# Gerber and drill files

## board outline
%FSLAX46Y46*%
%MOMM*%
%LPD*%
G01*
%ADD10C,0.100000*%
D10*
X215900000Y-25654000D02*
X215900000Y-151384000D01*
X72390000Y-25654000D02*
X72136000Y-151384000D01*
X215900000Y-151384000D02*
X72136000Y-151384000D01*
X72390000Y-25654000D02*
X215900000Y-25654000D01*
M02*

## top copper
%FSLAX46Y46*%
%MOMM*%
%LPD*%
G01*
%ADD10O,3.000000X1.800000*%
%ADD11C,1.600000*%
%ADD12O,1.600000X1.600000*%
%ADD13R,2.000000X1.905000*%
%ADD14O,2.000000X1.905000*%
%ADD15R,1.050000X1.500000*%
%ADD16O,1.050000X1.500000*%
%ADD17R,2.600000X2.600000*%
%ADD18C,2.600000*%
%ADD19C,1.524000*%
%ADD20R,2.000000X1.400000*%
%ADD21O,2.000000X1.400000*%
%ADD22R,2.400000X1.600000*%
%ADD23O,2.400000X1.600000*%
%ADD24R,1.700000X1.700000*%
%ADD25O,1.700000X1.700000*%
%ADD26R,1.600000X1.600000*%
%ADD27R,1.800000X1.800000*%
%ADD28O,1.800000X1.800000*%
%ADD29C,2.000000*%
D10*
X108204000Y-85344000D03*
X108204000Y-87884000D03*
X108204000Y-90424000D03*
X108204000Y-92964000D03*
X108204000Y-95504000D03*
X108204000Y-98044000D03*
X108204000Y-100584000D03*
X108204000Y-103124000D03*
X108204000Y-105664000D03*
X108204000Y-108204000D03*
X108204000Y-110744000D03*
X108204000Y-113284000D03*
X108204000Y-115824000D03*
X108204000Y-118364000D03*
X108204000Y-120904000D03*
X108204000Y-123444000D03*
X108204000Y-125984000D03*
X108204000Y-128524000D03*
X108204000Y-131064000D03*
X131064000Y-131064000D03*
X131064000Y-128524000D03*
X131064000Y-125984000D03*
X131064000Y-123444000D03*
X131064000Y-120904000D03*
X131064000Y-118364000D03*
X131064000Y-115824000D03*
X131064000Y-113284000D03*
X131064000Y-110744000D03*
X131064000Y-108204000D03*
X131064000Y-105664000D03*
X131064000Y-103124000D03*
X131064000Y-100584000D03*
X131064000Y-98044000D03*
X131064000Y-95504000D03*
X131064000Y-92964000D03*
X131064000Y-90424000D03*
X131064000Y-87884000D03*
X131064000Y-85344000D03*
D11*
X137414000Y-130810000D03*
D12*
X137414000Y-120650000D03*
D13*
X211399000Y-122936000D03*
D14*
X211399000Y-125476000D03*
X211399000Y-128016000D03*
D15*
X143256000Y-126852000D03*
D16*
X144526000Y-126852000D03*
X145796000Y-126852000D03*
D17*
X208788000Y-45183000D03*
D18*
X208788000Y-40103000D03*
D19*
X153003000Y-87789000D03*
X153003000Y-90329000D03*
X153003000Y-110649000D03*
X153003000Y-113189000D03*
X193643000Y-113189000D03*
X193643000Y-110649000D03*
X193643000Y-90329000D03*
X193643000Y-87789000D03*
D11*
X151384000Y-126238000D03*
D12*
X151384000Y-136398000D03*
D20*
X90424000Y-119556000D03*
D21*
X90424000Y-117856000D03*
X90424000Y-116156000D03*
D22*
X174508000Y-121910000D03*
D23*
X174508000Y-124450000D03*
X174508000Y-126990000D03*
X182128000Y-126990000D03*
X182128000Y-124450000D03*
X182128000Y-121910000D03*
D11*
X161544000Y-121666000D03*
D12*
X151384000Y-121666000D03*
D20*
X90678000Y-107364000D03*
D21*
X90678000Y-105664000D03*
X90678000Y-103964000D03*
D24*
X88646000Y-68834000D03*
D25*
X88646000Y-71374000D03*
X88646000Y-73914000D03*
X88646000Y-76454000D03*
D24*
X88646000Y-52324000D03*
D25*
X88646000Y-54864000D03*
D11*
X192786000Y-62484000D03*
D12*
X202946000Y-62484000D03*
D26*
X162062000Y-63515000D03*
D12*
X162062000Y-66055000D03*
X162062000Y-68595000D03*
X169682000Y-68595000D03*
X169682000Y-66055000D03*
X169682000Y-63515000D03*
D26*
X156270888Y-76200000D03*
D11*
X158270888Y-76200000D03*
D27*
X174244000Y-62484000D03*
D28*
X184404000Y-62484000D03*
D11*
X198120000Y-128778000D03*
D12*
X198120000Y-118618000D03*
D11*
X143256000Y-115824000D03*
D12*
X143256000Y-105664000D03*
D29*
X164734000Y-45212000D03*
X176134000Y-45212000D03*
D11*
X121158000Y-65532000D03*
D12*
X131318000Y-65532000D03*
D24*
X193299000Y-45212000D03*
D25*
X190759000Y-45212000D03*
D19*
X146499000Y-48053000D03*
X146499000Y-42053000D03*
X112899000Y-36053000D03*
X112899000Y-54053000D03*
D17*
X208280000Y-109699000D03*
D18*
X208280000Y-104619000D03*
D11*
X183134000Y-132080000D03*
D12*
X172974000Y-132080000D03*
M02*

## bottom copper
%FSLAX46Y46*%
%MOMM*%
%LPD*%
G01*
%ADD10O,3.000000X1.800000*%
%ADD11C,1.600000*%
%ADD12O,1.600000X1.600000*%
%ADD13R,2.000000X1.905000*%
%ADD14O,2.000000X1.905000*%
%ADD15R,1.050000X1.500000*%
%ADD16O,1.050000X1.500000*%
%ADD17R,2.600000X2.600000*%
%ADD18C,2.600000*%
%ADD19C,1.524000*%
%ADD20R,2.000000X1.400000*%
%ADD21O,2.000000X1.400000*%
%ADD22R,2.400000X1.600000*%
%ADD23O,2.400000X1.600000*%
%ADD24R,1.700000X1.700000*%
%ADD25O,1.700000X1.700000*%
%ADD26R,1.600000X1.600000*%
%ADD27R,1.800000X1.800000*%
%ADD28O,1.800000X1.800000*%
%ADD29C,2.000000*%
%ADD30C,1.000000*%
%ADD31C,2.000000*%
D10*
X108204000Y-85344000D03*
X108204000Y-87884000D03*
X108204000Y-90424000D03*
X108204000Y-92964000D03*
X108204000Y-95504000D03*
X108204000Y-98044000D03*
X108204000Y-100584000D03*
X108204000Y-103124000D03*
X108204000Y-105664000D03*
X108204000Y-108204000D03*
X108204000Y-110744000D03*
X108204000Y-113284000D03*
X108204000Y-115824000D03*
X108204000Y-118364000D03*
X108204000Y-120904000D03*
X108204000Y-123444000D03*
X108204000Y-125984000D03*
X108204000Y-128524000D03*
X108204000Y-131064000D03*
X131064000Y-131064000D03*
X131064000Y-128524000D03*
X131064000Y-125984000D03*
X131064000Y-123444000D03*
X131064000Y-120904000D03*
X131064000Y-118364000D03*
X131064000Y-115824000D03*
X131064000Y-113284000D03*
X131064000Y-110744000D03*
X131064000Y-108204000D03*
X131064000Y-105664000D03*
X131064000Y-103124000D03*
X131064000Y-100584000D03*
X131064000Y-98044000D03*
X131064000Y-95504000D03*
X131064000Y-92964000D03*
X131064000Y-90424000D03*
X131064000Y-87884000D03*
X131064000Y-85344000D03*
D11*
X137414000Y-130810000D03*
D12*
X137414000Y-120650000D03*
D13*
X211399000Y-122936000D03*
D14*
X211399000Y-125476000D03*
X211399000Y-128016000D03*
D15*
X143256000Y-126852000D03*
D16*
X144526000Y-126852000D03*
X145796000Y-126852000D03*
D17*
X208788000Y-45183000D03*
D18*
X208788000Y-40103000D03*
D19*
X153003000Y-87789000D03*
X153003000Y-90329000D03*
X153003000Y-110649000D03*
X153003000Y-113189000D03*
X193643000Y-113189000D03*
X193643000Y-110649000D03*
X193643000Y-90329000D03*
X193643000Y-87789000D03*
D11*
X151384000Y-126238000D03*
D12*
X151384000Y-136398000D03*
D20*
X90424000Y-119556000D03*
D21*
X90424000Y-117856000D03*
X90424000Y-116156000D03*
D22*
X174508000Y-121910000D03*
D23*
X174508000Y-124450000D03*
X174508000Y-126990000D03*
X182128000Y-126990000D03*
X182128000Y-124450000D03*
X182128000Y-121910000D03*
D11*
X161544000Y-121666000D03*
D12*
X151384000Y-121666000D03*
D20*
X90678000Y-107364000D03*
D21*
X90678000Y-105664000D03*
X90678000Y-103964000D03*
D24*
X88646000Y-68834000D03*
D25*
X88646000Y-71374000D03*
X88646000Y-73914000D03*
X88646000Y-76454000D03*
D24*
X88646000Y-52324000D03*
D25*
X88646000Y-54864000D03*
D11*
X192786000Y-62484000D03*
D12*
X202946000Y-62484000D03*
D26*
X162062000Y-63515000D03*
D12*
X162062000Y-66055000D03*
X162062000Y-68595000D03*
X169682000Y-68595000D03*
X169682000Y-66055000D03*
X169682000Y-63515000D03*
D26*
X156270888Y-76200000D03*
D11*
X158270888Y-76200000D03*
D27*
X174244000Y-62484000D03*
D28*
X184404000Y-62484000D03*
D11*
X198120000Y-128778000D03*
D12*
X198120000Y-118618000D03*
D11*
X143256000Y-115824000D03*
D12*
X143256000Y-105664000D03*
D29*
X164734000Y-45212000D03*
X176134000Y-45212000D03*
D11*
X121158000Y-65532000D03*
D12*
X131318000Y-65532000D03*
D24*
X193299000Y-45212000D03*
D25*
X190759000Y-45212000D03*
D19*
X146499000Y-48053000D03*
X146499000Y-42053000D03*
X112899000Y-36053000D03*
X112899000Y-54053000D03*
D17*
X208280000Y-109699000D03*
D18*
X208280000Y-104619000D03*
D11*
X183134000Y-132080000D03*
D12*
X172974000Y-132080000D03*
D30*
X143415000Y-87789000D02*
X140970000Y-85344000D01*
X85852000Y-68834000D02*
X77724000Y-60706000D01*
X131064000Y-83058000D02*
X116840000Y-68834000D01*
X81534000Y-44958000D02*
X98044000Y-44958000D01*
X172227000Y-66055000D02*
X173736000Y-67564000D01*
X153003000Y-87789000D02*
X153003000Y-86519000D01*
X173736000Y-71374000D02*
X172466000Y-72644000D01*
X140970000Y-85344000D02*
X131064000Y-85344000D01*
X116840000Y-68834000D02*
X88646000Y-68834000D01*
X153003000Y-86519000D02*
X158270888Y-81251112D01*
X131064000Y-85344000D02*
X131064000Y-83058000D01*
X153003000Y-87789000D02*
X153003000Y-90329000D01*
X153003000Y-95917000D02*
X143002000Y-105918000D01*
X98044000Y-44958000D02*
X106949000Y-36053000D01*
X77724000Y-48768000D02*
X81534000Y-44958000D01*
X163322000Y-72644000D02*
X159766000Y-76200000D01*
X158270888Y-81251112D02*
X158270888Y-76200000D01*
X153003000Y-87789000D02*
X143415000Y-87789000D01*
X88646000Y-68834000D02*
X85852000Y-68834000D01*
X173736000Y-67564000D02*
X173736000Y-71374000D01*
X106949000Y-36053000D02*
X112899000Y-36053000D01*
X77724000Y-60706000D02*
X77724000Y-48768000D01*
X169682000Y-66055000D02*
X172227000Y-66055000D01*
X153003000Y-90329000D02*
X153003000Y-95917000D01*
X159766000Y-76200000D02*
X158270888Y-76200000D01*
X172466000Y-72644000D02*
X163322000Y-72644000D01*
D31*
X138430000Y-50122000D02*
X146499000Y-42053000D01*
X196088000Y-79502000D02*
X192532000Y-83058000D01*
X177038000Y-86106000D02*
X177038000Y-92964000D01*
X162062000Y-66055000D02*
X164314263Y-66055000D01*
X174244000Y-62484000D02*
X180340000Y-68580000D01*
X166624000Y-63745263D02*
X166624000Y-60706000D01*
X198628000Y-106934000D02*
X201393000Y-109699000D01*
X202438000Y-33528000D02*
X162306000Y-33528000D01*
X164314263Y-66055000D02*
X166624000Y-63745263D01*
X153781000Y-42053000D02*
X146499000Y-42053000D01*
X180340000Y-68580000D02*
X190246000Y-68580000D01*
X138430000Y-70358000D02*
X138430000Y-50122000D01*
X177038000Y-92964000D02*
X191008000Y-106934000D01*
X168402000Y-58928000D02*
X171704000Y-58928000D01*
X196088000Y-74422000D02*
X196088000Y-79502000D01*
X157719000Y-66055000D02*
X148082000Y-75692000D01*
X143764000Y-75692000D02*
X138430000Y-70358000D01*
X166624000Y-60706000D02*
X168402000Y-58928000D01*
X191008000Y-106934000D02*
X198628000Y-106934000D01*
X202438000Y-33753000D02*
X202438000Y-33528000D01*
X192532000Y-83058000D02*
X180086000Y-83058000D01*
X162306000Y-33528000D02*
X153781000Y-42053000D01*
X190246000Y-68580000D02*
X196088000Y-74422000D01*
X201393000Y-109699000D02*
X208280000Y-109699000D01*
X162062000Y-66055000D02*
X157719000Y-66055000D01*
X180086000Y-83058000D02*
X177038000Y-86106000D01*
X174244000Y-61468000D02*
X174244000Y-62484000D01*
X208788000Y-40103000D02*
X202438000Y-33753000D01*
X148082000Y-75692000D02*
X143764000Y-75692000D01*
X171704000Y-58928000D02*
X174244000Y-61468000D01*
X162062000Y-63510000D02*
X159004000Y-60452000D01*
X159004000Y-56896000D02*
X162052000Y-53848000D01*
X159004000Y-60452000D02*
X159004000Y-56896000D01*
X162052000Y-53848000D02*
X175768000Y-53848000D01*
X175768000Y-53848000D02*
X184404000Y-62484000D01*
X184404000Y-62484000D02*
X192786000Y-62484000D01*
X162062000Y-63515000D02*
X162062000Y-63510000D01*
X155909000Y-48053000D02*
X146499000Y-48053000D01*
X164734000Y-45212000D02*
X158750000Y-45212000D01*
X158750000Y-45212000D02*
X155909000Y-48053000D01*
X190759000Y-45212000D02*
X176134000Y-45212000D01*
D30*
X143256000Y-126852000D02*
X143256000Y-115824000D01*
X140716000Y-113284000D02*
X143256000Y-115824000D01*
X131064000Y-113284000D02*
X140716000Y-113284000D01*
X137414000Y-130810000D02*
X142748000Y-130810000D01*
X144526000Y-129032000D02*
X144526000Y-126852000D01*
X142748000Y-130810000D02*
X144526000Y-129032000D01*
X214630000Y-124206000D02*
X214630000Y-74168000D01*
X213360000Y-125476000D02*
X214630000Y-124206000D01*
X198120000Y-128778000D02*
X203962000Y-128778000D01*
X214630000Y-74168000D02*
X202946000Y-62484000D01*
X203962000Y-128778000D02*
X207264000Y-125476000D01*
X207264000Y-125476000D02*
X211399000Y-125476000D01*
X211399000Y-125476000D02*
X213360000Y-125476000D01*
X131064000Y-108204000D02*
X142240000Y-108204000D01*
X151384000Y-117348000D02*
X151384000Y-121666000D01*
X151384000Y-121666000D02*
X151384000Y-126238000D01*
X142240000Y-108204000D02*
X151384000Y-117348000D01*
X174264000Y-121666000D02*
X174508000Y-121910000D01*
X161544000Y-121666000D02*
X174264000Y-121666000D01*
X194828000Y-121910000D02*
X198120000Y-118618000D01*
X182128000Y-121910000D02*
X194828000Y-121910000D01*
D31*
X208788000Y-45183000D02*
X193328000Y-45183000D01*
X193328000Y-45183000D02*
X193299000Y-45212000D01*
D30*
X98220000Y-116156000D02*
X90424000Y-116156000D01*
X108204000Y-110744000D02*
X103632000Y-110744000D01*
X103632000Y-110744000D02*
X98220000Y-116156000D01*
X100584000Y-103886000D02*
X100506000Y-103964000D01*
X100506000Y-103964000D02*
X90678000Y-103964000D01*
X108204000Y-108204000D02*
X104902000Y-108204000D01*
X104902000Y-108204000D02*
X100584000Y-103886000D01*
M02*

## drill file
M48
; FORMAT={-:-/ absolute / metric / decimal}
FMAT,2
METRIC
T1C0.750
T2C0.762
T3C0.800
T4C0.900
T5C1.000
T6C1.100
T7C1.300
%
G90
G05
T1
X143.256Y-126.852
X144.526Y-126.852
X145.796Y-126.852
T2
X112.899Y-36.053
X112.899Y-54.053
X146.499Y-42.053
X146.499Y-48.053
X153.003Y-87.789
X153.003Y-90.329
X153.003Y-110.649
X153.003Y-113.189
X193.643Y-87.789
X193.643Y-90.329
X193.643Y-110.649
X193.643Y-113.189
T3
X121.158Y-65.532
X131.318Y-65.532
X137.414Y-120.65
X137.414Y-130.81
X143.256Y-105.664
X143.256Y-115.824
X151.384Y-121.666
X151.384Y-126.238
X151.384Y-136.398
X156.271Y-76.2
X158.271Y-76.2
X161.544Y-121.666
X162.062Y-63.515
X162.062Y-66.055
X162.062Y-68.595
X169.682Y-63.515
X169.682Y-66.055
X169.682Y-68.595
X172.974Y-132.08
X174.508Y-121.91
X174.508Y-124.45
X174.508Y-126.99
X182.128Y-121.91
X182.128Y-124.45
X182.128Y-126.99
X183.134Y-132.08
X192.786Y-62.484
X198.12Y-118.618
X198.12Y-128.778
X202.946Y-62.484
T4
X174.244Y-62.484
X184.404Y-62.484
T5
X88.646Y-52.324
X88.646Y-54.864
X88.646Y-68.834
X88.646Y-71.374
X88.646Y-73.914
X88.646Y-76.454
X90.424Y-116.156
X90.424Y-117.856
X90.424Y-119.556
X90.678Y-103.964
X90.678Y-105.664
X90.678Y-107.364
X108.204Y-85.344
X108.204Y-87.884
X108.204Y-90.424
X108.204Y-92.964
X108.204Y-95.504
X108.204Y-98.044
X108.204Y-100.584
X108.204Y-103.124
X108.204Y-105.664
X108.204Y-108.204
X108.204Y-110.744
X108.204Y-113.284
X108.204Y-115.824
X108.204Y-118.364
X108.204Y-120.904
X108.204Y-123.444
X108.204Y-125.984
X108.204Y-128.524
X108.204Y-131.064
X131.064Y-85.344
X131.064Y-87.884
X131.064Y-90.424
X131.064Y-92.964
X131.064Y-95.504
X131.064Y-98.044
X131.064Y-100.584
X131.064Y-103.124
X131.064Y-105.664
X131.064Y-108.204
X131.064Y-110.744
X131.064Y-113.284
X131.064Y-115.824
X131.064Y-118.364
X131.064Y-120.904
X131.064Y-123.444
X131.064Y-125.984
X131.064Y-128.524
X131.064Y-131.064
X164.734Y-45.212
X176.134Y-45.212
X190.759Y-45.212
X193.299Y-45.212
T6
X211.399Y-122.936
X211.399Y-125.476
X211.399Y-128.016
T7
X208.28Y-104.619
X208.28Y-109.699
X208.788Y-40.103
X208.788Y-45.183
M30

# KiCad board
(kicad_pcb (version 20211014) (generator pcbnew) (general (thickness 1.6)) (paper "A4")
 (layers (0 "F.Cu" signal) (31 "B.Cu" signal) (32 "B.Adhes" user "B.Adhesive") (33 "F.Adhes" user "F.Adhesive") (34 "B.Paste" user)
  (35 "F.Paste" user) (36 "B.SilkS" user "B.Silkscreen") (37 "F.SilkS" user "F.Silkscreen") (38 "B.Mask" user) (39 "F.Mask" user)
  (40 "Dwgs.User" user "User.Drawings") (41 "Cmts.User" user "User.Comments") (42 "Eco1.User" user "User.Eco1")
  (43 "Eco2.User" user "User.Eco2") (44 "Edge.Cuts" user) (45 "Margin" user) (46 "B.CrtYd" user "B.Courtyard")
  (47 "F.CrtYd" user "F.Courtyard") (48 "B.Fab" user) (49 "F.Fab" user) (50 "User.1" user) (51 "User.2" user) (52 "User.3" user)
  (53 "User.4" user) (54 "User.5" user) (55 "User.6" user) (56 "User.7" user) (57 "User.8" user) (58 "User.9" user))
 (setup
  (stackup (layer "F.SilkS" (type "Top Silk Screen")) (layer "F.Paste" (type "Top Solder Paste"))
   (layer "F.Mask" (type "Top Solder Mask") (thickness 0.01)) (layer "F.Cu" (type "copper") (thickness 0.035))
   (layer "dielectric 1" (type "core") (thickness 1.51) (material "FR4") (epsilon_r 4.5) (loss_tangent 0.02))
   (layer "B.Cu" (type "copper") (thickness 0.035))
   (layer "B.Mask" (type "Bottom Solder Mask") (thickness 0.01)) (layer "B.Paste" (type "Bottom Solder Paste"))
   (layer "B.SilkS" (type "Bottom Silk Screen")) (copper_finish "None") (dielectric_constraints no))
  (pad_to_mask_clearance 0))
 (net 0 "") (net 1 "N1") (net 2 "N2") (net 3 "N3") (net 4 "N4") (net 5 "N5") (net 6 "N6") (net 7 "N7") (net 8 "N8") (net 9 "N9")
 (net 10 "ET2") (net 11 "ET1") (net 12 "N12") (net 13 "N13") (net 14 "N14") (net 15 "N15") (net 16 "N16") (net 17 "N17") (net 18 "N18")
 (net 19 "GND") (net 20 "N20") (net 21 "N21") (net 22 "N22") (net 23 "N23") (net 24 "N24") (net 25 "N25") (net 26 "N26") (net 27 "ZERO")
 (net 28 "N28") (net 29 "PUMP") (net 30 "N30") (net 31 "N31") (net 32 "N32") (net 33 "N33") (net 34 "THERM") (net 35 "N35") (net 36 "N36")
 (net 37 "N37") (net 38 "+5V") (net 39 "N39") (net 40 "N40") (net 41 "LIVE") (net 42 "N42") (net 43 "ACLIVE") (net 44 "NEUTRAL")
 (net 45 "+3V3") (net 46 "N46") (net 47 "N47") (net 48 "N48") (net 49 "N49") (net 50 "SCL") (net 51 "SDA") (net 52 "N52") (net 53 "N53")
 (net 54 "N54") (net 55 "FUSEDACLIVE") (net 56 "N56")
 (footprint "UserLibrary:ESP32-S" (layer "F.Cu") (at 119.634 108.204)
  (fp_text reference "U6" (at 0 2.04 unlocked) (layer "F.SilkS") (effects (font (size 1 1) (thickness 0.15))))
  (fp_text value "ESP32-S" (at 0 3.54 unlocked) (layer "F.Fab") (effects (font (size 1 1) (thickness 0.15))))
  (pad "1" thru_hole oval (at -11.43 -22.86) (size 3 1.8) (drill 1) (layers *.Cu *.Mask) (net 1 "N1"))
  (pad "2" thru_hole oval (at -11.43 -20.32) (size 3 1.8) (drill 1) (layers *.Cu *.Mask) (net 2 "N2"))
  (pad "3" thru_hole oval (at -11.43 -17.78) (size 3 1.8) (drill 1) (layers *.Cu *.Mask) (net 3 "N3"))
  (pad "4" thru_hole oval (at -11.43 -15.24) (size 3 1.8) (drill 1) (layers *.Cu *.Mask) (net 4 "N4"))
  (pad "5" thru_hole oval (at -11.43 -12.7) (size 3 1.8) (drill 1) (layers *.Cu *.Mask) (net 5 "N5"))
  (pad "6" thru_hole oval (at -11.43 -10.16) (size 3 1.8) (drill 1) (layers *.Cu *.Mask) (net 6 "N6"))
  (pad "7" thru_hole oval (at -11.43 -7.62) (size 3 1.8) (drill 1) (layers *.Cu *.Mask) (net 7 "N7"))
  (pad "8" thru_hole oval (at -11.43 -5.08) (size 3 1.8) (drill 1) (layers *.Cu *.Mask) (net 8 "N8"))
  (pad "9" thru_hole oval (at -11.43 -2.54) (size 3 1.8) (drill 1) (layers *.Cu *.Mask) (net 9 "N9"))
  (pad "10" thru_hole oval (at -11.43 0) (size 3 1.8) (drill 1) (layers *.Cu *.Mask) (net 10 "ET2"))
  (pad "11" thru_hole oval (at -11.43 2.54) (size 3 1.8) (drill 1) (layers *.Cu *.Mask) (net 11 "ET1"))
  (pad "12" thru_hole oval (at -11.43 5.08) (size 3 1.8) (drill 1) (layers *.Cu *.Mask) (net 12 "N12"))
  (pad "13" thru_hole oval (at -11.43 7.62) (size 3 1.8) (drill 1) (layers *.Cu *.Mask) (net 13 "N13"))
  (pad "14" thru_hole oval (at -11.43 10.16) (size 3 1.8) (drill 1) (layers *.Cu *.Mask) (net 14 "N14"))
  (pad "15" thru_hole oval (at -11.43 12.7) (size 3 1.8) (drill 1) (layers *.Cu *.Mask) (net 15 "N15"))
  (pad "16" thru_hole oval (at -11.43 15.24) (size 3 1.8) (drill 1) (layers *.Cu *.Mask) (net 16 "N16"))
  (pad "17" thru_hole oval (at -11.43 17.78) (size 3 1.8) (drill 1) (layers *.Cu *.Mask) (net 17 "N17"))
  (pad "18" thru_hole oval (at -11.43 20.32) (size 3 1.8) (drill 1) (layers *.Cu *.Mask) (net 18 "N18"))
  (pad "19" thru_hole oval (at -11.43 22.86) (size 3 1.8) (drill 1) (layers *.Cu *.Mask) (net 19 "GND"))
  (pad "20" thru_hole oval (at 11.43 22.86) (size 3 1.8) (drill 1) (layers *.Cu *.Mask) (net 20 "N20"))
  (pad "21" thru_hole oval (at 11.43 20.32) (size 3 1.8) (drill 1) (layers *.Cu *.Mask) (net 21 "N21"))
  (pad "22" thru_hole oval (at 11.43 17.78) (size 3 1.8) (drill 1) (layers *.Cu *.Mask) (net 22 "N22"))
  (pad "23" thru_hole oval (at 11.43 15.24) (size 3 1.8) (drill 1) (layers *.Cu *.Mask) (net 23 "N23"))
  (pad "24" thru_hole oval (at 11.43 12.7) (size 3 1.8) (drill 1) (layers *.Cu *.Mask) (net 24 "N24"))
  (pad "25" thru_hole oval (at 11.43 10.16) (size 3 1.8) (drill 1) (layers *.Cu *.Mask) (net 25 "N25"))
  (pad "26" thru_hole oval (at 11.43 7.62) (size 3 1.8) (drill 1) (layers *.Cu *.Mask) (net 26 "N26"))
  (pad "27" thru_hole oval (at 11.43 5.08) (size 3 1.8) (drill 1) (layers *.Cu *.Mask) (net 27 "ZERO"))
  (pad "28" thru_hole oval (at 11.43 2.54) (size 3 1.8) (drill 1) (layers *.Cu *.Mask) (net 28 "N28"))
  (pad "29" thru_hole oval (at 11.43 0) (size 3 1.8) (drill 1) (layers *.Cu *.Mask) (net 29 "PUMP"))
  (pad "30" thru_hole oval (at 11.43 -2.54) (size 3 1.8) (drill 1) (layers *.Cu *.Mask) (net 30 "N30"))
  (pad "31" thru_hole oval (at 11.43 -5.08) (size 3 1.8) (drill 1) (layers *.Cu *.Mask) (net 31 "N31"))
  (pad "32" thru_hole oval (at 11.43 -7.62) (size 3 1.8) (drill 1) (layers *.Cu *.Mask) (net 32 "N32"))
  (pad "33" thru_hole oval (at 11.43 -10.16) (size 3 1.8) (drill 1) (layers *.Cu *.Mask) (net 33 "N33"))
  (pad "34" thru_hole oval (at 11.43 -12.7) (size 3 1.8) (drill 1) (layers *.Cu *.Mask) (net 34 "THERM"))
  (pad "35" thru_hole oval (at 11.43 -15.24) (size 3 1.8) (drill 1) (layers *.Cu *.Mask) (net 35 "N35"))
  (pad "36" thru_hole oval (at 11.43 -17.78) (size 3 1.8) (drill 1) (layers *.Cu *.Mask) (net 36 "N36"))
  (pad "37" thru_hole oval (at 11.43 -20.32) (size 3 1.8) (drill 1) (layers *.Cu *.Mask) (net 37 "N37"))
  (pad "38" thru_hole oval (at 11.43 -22.86) (size 3 1.8) (drill 1) (layers *.Cu *.Mask) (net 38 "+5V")))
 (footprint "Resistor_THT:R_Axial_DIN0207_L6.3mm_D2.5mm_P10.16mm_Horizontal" (layer "F.Cu") (at 137.414 130.81 90)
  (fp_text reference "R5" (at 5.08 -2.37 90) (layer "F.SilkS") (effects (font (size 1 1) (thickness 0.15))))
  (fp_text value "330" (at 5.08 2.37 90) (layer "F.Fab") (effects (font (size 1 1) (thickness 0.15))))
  (pad "1" thru_hole circle (at 0 0 90) (size 1.6 1.6) (drill 0.8) (layers *.Cu *.Mask) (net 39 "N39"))
  (pad "2" thru_hole oval (at 10.16 0 90) (size 1.6 1.6) (drill 0.8) (layers *.Cu *.Mask) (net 19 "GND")))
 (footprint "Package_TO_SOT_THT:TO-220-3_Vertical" (layer "F.Cu") (at 211.399 122.936 -90)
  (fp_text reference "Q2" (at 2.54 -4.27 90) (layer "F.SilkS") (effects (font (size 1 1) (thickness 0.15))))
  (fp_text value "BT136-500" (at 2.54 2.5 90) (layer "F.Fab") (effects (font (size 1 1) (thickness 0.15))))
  (pad "1" thru_hole rect (at 0 0 270) (size 1.905 2) (drill 1.1) (layers *.Cu *.Mask) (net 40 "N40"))
  (pad "2" thru_hole oval (at 2.54 0 270) (size 1.905 2) (drill 1.1) (layers *.Cu *.Mask) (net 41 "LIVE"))
  (pad "3" thru_hole oval (at 5.08 0 270) (size 1.905 2) (drill 1.1) (layers *.Cu *.Mask) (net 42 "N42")))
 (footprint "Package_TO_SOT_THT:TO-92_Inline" (layer "F.Cu") (at 143.256 126.852)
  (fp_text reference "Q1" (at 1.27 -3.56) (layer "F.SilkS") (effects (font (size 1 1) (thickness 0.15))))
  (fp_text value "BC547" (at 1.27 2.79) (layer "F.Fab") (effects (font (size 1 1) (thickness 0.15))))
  (pad "1" thru_hole rect (at 0 0) (size 1.05 1.5) (drill 0.75) (layers *.Cu *.Mask) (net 27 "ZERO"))
  (pad "2" thru_hole oval (at 1.27 0) (size 1.05 1.5) (drill 0.75) (layers *.Cu *.Mask) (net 39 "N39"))
  (pad "3" thru_hole oval (at 2.54 0) (size 1.05 1.5) (drill 0.75) (layers *.Cu *.Mask) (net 19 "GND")))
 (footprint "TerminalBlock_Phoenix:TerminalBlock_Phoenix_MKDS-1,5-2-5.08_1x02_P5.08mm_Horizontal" (layer "F.Cu") (at 208.788 45.183 90)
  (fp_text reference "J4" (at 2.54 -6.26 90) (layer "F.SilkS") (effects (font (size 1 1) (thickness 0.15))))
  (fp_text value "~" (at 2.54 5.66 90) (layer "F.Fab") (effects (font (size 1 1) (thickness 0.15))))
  (pad "1" thru_hole rect (at 0 0 90) (size 2.6 2.6) (drill 1.3) (layers *.Cu *.Mask) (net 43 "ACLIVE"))
  (pad "2" thru_hole circle (at 5.08 0 90) (size 2.6 2.6) (drill 1.3) (layers *.Cu *.Mask) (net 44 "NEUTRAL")))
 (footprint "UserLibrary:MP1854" (layer "F.Cu") (at 150.463 115.729)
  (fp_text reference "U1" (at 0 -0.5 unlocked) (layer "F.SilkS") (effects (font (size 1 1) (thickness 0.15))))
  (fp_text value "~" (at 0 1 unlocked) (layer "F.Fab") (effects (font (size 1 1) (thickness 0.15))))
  (pad "1" thru_hole circle (at 2.54 -27.94) (size 1.524 1.524) (drill 0.762) (layers *.Cu *.Mask) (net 38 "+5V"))
  (pad "2" thru_hole circle (at 2.54 -25.4) (size 1.524 1.524) (drill 0.762) (layers *.Cu *.Mask) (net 38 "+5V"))
  (pad "3" thru_hole circle (at 2.54 -5.08) (size 1.524 1.524) (drill 0.762) (layers *.Cu *.Mask) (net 19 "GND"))
  (pad "4" thru_hole circle (at 2.54 -2.54) (size 1.524 1.524) (drill 0.762) (layers *.Cu *.Mask) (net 19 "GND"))
  (pad "5" thru_hole circle (at 43.18 -2.54) (size 1.524 1.524) (drill 0.762) (layers *.Cu *.Mask) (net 19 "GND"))
  (pad "6" thru_hole circle (at 43.18 -5.08) (size 1.524 1.524) (drill 0.762) (layers *.Cu *.Mask) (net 19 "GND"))
  (pad "7" thru_hole circle (at 43.18 -25.4) (size 1.524 1.524) (drill 0.762) (layers *.Cu *.Mask) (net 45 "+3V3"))
  (pad "8" thru_hole circle (at 43.18 -27.94) (size 1.524 1.524) (drill 0.762) (layers *.Cu *.Mask) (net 45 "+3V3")))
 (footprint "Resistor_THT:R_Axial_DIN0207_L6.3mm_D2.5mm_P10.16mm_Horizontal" (layer "F.Cu") (at 151.384 126.238 -90)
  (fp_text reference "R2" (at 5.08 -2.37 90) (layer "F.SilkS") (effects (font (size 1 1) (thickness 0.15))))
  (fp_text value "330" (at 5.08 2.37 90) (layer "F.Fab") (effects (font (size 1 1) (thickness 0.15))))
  (pad "1" thru_hole circle (at 0 0 270) (size 1.6 1.6) (drill 0.8) (layers *.Cu *.Mask) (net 29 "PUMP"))
  (pad "2" thru_hole oval (at 10.16 0 270) (size 1.6 1.6) (drill 0.8) (layers *.Cu *.Mask) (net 19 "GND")))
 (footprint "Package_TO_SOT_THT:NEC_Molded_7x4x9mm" (layer "F.Cu") (at 90.424 119.556 90)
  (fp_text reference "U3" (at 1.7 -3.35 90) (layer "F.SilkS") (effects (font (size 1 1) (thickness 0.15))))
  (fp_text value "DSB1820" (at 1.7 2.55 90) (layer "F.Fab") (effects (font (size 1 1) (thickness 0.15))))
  (pad "1" thru_hole rect (at 0 0 270) (size 1.4 2) (drill 1) (layers *.Cu *.Mask) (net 45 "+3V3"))
  (pad "2" thru_hole oval (at 1.7 0 270) (size 1.4 2) (drill 1) (layers *.Cu *.Mask) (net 19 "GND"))
  (pad "3" thru_hole oval (at 3.4 0 270) (size 1.4 2) (drill 1) (layers *.Cu *.Mask) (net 11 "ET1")))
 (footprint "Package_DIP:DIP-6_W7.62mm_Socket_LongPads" (layer "F.Cu") (at 174.508 121.91)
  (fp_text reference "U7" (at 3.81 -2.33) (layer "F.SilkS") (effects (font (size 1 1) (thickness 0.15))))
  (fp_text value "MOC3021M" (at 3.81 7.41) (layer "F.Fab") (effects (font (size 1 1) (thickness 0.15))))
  (pad "1" thru_hole rect (at 0 0) (size 2.4 1.6) (drill 0.8) (layers *.Cu *.Mask) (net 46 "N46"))
  (pad "2" thru_hole oval (at 0 2.54) (size 2.4 1.6) (drill 0.8) (layers *.Cu *.Mask) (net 19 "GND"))
  (pad "3" thru_hole oval (at 0 5.08) (size 2.4 1.6) (drill 0.8) (layers *.Cu *.Mask) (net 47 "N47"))
  (pad "4" thru_hole oval (at 7.62 5.08) (size 2.4 1.6) (drill 0.8) (layers *.Cu *.Mask) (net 42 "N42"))
  (pad "5" thru_hole oval (at 7.62 2.54) (size 2.4 1.6) (drill 0.8) (layers *.Cu *.Mask) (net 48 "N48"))
  (pad "6" thru_hole oval (at 7.62 0) (size 2.4 1.6) (drill 0.8) (layers *.Cu *.Mask) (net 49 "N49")))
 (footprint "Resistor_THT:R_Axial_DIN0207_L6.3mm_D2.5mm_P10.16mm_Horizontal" (layer "F.Cu") (at 161.544 121.666 180)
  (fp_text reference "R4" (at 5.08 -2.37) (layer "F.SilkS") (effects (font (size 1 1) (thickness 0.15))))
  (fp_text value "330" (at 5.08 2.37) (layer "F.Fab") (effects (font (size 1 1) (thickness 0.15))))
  (pad "1" thru_hole circle (at 0 0 180) (size 1.6 1.6) (drill 0.8) (layers *.Cu *.Mask) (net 46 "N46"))
  (pad "2" thru_hole oval (at 10.16 0 180) (size 1.6 1.6) (drill 0.8) (layers *.Cu *.Mask) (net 29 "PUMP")))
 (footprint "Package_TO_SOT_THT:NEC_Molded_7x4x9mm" (layer "F.Cu") (at 90.678 107.364 90)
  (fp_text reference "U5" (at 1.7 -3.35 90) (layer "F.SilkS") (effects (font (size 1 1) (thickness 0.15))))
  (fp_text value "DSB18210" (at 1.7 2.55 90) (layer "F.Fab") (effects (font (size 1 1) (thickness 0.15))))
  (pad "1" thru_hole rect (at 0 0 270) (size 1.4 2) (drill 1) (layers *.Cu *.Mask) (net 45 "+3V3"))
  (pad "2" thru_hole oval (at 1.7 0 270) (size 1.4 2) (drill 1) (layers *.Cu *.Mask) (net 19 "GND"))
  (pad "3" thru_hole oval (at 3.4 0 270) (size 1.4 2) (drill 1) (layers *.Cu *.Mask) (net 10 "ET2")))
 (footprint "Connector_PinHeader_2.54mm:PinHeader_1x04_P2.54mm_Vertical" (layer "F.Cu") (at 88.646 68.834)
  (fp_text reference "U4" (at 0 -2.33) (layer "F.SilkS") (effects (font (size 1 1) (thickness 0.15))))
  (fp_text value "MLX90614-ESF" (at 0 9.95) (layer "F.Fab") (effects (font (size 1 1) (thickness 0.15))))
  (pad "1" thru_hole rect (at 0 0) (size 1.7 1.7) (drill 1) (layers *.Cu *.Mask) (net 38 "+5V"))
  (pad "2" thru_hole oval (at 0 2.54) (size 1.7 1.7) (drill 1) (layers *.Cu *.Mask) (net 19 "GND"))
  (pad "3" thru_hole oval (at 0 5.08) (size 1.7 1.7) (drill 1) (layers *.Cu *.Mask) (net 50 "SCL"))
  (pad "4" thru_hole oval (at 0 7.62) (size 1.7 1.7) (drill 1) (layers *.Cu *.Mask) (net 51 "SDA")))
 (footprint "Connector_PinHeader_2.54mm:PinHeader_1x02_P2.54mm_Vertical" (layer "F.Cu") (at 88.646 52.324)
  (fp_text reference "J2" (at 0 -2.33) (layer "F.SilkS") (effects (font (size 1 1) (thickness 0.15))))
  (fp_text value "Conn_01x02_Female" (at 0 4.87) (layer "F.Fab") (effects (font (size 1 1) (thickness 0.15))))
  (pad "1" thru_hole rect (at 0 0) (size 1.7 1.7) (drill 1) (layers *.Cu *.Mask) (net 34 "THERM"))
  (pad "2" thru_hole oval (at 0 2.54) (size 1.7 1.7) (drill 1) (layers *.Cu *.Mask) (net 19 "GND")))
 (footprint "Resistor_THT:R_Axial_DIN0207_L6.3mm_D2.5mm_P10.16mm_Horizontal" (layer "F.Cu") (at 192.786 62.484)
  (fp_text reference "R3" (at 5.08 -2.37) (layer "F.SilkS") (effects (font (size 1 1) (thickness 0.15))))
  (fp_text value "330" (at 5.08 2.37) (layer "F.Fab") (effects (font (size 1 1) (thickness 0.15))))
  (pad "1" thru_hole circle (at 0 0) (size 1.6 1.6) (drill 0.8) (layers *.Cu *.Mask) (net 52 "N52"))
  (pad "2" thru_hole oval (at 10.16 0) (size 1.6 1.6) (drill 0.8) (layers *.Cu *.Mask) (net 41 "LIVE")))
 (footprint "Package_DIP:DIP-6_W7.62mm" (layer "F.Cu") (at 162.062 63.515)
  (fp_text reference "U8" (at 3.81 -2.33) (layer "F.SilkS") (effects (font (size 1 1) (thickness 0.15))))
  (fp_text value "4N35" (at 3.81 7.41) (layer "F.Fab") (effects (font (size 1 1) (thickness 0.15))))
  (pad "1" thru_hole rect (at 0 0) (size 1.6 1.6) (drill 0.8) (layers *.Cu *.Mask) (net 52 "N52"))
  (pad "2" thru_hole oval (at 0 2.54) (size 1.6 1.6) (drill 0.8) (layers *.Cu *.Mask) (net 44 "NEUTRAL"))
  (pad "3" thru_hole oval (at 0 5.08) (size 1.6 1.6) (drill 0.8) (layers *.Cu *.Mask) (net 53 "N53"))
  (pad "4" thru_hole oval (at 7.62 5.08) (size 1.6 1.6) (drill 0.8) (layers *.Cu *.Mask) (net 39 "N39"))
  (pad "5" thru_hole oval (at 7.62 2.54) (size 1.6 1.6) (drill 0.8) (layers *.Cu *.Mask) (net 38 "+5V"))
  (pad "6" thru_hole oval (at 7.62 0) (size 1.6 1.6) (drill 0.8) (layers *.Cu *.Mask) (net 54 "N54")))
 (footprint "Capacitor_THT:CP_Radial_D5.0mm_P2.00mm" (layer "F.Cu") (at 156.270888 76.2)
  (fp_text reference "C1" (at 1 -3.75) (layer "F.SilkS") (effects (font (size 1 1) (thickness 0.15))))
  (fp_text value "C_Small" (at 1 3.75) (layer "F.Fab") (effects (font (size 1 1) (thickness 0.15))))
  (pad "1" thru_hole rect (at 0 0) (size 1.6 1.6) (drill 0.8) (layers *.Cu *.Mask) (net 19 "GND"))
  (pad "2" thru_hole circle (at 2 0) (size 1.6 1.6) (drill 0.8) (layers *.Cu *.Mask) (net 38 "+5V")))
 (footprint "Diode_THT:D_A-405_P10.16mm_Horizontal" (layer "F.Cu") (at 174.244 62.484)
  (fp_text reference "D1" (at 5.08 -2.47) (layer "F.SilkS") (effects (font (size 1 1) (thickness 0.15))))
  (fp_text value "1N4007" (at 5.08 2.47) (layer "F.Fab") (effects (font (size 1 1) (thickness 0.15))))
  (pad "1" thru_hole rect (at 0 0) (size 1.8 1.8) (drill 0.9) (layers *.Cu *.Mask) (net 44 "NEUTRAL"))
  (pad "2" thru_hole oval (at 10.16 0) (size 1.8 1.8) (drill 0.9) (layers *.Cu *.Mask) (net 52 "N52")))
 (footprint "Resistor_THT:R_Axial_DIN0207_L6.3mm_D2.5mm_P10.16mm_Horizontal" (layer "F.Cu") (at 198.12 128.778 90)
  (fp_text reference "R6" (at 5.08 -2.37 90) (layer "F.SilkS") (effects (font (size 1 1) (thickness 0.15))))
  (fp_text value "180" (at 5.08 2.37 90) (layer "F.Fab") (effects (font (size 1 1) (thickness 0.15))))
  (pad "1" thru_hole circle (at 0 0 90) (size 1.6 1.6) (drill 0.8) (layers *.Cu *.Mask) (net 41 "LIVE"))
  (pad "2" thru_hole oval (at 10.16 0 90) (size 1.6 1.6) (drill 0.8) (layers *.Cu *.Mask) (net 49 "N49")))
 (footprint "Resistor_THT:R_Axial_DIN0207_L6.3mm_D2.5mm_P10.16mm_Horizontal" (layer "F.Cu") (at 143.256 115.824 90)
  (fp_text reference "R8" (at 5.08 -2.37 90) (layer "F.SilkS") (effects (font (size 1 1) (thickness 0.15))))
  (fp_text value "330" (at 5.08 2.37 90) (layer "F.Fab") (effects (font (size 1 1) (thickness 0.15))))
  (pad "1" thru_hole circle (at 0 0 90) (size 1.6 1.6) (drill 0.8) (layers *.Cu *.Mask) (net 27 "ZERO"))
  (pad "2" thru_hole oval (at 10.16 0 90) (size 1.6 1.6) (drill 0.8) (layers *.Cu *.Mask) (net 38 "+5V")))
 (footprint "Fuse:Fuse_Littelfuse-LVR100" (layer "F.Cu") (at 164.734 45.212)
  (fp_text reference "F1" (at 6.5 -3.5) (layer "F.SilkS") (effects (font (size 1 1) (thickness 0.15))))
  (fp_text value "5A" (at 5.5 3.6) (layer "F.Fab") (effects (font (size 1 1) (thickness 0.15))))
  (pad "1" thru_hole circle (at 0 0) (size 2 2) (drill 1) (layers *.Cu *.Mask) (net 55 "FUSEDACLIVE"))
  (pad "2" thru_hole circle (at 11.4 0) (size 2 2) (drill 1) (layers *.Cu *.Mask) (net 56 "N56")))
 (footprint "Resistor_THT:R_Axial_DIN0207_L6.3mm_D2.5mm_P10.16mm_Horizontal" (layer "F.Cu") (at 121.158 65.532)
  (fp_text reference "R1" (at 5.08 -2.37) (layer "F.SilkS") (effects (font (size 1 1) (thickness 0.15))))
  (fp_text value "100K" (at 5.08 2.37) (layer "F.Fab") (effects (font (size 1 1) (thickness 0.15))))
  (pad "1" thru_hole circle (at 0 0) (size 1.6 1.6) (drill 0.8) (layers *.Cu *.Mask) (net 45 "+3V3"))
  (pad "2" thru_hole oval (at 10.16 0) (size 1.6 1.6) (drill 0.8) (layers *.Cu *.Mask) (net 34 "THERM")))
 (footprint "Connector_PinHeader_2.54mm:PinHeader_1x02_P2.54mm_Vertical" (layer "F.Cu") (at 193.299 45.212 -90)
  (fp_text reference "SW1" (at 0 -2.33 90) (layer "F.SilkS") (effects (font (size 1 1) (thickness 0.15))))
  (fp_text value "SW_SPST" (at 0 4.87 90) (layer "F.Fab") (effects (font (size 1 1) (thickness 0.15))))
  (pad "1" thru_hole rect (at 0 0 270) (size 1.7 1.7) (drill 1) (layers *.Cu *.Mask) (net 43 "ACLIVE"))
  (pad "2" thru_hole oval (at 0 2.54 270) (size 1.7 1.7) (drill 1) (layers *.Cu *.Mask) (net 56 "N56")))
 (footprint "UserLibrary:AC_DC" (layer "F.Cu") (at 148.699 33.553 180)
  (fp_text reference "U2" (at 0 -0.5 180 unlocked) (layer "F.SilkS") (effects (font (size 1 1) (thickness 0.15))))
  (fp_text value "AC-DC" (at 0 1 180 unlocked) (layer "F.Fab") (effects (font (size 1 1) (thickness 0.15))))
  (pad "1" thru_hole circle (at 2.2 -14.5 180) (size 1.524 1.524) (drill 0.762) (layers *.Cu *.Mask) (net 55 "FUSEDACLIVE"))
  (pad "2" thru_hole circle (at 2.2 -8.5 180) (size 1.524 1.524) (drill 0.762) (layers *.Cu *.Mask) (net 44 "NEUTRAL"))
  (pad "3" thru_hole circle (at 35.8 -2.5 180) (size 1.524 1.524) (drill 0.762) (layers *.Cu *.Mask) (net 38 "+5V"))
  (pad "4" thru_hole circle (at 35.8 -20.5 180) (size 1.524 1.524) (drill 0.762) (layers *.Cu *.Mask) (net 19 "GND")))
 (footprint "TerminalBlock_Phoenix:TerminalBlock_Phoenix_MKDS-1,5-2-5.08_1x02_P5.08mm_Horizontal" (layer "F.Cu") (at 208.28 109.699 90)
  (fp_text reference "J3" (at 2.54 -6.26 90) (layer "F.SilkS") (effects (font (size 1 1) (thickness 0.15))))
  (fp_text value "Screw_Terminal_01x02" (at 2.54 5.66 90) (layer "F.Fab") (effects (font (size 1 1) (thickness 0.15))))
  (pad "1" thru_hole rect (at 0 0 90) (size 2.6 2.6) (drill 1.3) (layers *.Cu *.Mask) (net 44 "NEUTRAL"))
  (pad "2" thru_hole circle (at 5.08 0 90) (size 2.6 2.6) (drill 1.3) (layers *.Cu *.Mask) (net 40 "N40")))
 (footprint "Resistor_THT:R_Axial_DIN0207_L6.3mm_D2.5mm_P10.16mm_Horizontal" (layer "F.Cu") (at 183.134 132.08 180)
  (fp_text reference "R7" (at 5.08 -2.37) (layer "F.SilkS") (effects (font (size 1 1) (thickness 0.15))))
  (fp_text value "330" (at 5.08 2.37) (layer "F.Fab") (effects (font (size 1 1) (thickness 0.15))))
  (pad "1" thru_hole circle (at 0 0 180) (size 1.6 1.6) (drill 0.8) (layers *.Cu *.Mask) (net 42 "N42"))
  (pad "2" thru_hole oval (at 10.16 0 180) (size 1.6 1.6) (drill 0.8) (layers *.Cu *.Mask) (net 19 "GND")))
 (gr_line (start 215.9 25.654) (end 215.9 151.384) (layer "Edge.Cuts") (width 0.1))
 (gr_line (start 72.39 25.654) (end 72.136 151.384) (layer "Edge.Cuts") (width 0.1))
 (gr_line (start 215.9 151.384) (end 72.136 151.384) (layer "Edge.Cuts") (width 0.1))
 (gr_line (start 72.39 25.654) (end 215.9 25.654) (layer "Edge.Cuts") (width 0.1))
 (segment (start 143.415 87.789) (end 140.97 85.344) (width 1) (layer "B.Cu") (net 38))
 (segment (start 85.852 68.834) (end 77.724 60.706) (width 1) (layer "B.Cu") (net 38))
 (segment (start 131.064 83.058) (end 116.84 68.834) (width 1) (layer "B.Cu") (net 38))
 (segment (start 81.534 44.958) (end 98.044 44.958) (width 1) (layer "B.Cu") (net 38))
 (segment (start 172.227 66.055) (end 173.736 67.564) (width 1) (layer "B.Cu") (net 38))
 (segment (start 153.003 87.789) (end 153.003 86.519) (width 1) (layer "B.Cu") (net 38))
 (segment (start 173.736 71.374) (end 172.466 72.644) (width 1) (layer "B.Cu") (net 38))
 (segment (start 140.97 85.344) (end 131.064 85.344) (width 1) (layer "B.Cu") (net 38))
 (segment (start 116.84 68.834) (end 88.646 68.834) (width 1) (layer "B.Cu") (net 38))
 (segment (start 153.003 86.519) (end 158.270888 81.251112) (width 1) (layer "B.Cu") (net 38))
 (segment (start 131.064 85.344) (end 131.064 83.058) (width 1) (layer "B.Cu") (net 38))
 (segment (start 153.003 87.789) (end 153.003 90.329) (width 1) (layer "B.Cu") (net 38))
 (segment (start 153.003 95.917) (end 143.002 105.918) (width 1) (layer "B.Cu") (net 38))
 (segment (start 98.044 44.958) (end 106.949 36.053) (width 1) (layer "B.Cu") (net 38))
 (segment (start 77.724 48.768) (end 81.534 44.958) (width 1) (layer "B.Cu") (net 38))
 (segment (start 163.322 72.644) (end 159.766 76.2) (width 1) (layer "B.Cu") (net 38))
 (segment (start 158.270888 81.251112) (end 158.270888 76.2) (width 1) (layer "B.Cu") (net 38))
 (segment (start 153.003 87.789) (end 143.415 87.789) (width 1) (layer "B.Cu") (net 38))
 (segment (start 88.646 68.834) (end 85.852 68.834) (width 1) (layer "B.Cu") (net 38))
 (segment (start 173.736 67.564) (end 173.736 71.374) (width 1) (layer "B.Cu") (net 38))
 (segment (start 106.949 36.053) (end 112.899 36.053) (width 1) (layer "B.Cu") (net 38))
 (segment (start 77.724 60.706) (end 77.724 48.768) (width 1) (layer "B.Cu") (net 38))
 (segment (start 169.682 66.055) (end 172.227 66.055) (width 1) (layer "B.Cu") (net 38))
 (segment (start 153.003 90.329) (end 153.003 95.917) (width 1) (layer "B.Cu") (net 38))
 (segment (start 159.766 76.2) (end 158.270888 76.2) (width 1) (layer "B.Cu") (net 38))
 (segment (start 172.466 72.644) (end 163.322 72.644) (width 1) (layer "B.Cu") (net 38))
 (segment (start 138.43 50.122) (end 146.499 42.053) (width 2) (layer "B.Cu") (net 44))
 (segment (start 196.088 79.502) (end 192.532 83.058) (width 2) (layer "B.Cu") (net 44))
 (segment (start 177.038 86.106) (end 177.038 92.964) (width 2) (layer "B.Cu") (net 44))
 (segment (start 162.062 66.055) (end 164.314263 66.055) (width 2) (layer "B.Cu") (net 44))
 (segment (start 174.244 62.484) (end 180.34 68.58) (width 2) (layer "B.Cu") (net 44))
 (segment (start 166.624 63.745263) (end 166.624 60.706) (width 2) (layer "B.Cu") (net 44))
 (segment (start 198.628 106.934) (end 201.393 109.699) (width 2) (layer "B.Cu") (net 44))
 (segment (start 202.438 33.528) (end 162.306 33.528) (width 2) (layer "B.Cu") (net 44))
 (segment (start 164.314263 66.055) (end 166.624 63.745263) (width 2) (layer "B.Cu") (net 44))
 (segment (start 153.781 42.053) (end 146.499 42.053) (width 2) (layer "B.Cu") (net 44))
 (segment (start 180.34 68.58) (end 190.246 68.58) (width 2) (layer "B.Cu") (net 44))
 (segment (start 138.43 70.358) (end 138.43 50.122) (width 2) (layer "B.Cu") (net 44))
 (segment (start 177.038 92.964) (end 191.008 106.934) (width 2) (layer "B.Cu") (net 44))
 (segment (start 168.402 58.928) (end 171.704 58.928) (width 2) (layer "B.Cu") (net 44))
 (segment (start 196.088 74.422) (end 196.088 79.502) (width 2) (layer "B.Cu") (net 44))
 (segment (start 157.719 66.055) (end 148.082 75.692) (width 2) (layer "B.Cu") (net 44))
 (segment (start 143.764 75.692) (end 138.43 70.358) (width 2) (layer "B.Cu") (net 44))
 (segment (start 166.624 60.706) (end 168.402 58.928) (width 2) (layer "B.Cu") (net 44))
 (segment (start 191.008 106.934) (end 198.628 106.934) (width 2) (layer "B.Cu") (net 44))
 (segment (start 202.438 33.753) (end 202.438 33.528) (width 2) (layer "B.Cu") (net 44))
 (segment (start 192.532 83.058) (end 180.086 83.058) (width 2) (layer "B.Cu") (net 44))
 (segment (start 162.306 33.528) (end 153.781 42.053) (width 2) (layer "B.Cu") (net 44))
 (segment (start 190.246 68.58) (end 196.088 74.422) (width 2) (layer "B.Cu") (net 44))
 (segment (start 201.393 109.699) (end 208.28 109.699) (width 2) (layer "B.Cu") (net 44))
 (segment (start 162.062 66.055) (end 157.719 66.055) (width 2) (layer "B.Cu") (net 44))
 (segment (start 180.086 83.058) (end 177.038 86.106) (width 2) (layer "B.Cu") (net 44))
 (segment (start 174.244 61.468) (end 174.244 62.484) (width 2) (layer "B.Cu") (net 44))
 (segment (start 208.788 40.103) (end 202.438 33.753) (width 2) (layer "B.Cu") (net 44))
 (segment (start 148.082 75.692) (end 143.764 75.692) (width 2) (layer "B.Cu") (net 44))
 (segment (start 171.704 58.928) (end 174.244 61.468) (width 2) (layer "B.Cu") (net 44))
 (segment (start 162.062 63.51) (end 159.004 60.452) (width 2) (layer "B.Cu") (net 52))
 (segment (start 159.004 56.896) (end 162.052 53.848) (width 2) (layer "B.Cu") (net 52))
 (segment (start 159.004 60.452) (end 159.004 56.896) (width 2) (layer "B.Cu") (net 52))
 (segment (start 162.052 53.848) (end 175.768 53.848) (width 2) (layer "B.Cu") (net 52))
 (segment (start 175.768 53.848) (end 184.404 62.484) (width 2) (layer "B.Cu") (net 52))
 (segment (start 184.404 62.484) (end 192.786 62.484) (width 2) (layer "B.Cu") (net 52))
 (segment (start 162.062 63.515) (end 162.062 63.51) (width 2) (layer "B.Cu") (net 52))
 (segment (start 155.909 48.053) (end 146.499 48.053) (width 2) (layer "B.Cu") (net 55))
 (segment (start 164.734 45.212) (end 158.75 45.212) (width 2) (layer "B.Cu") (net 55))
 (segment (start 158.75 45.212) (end 155.909 48.053) (width 2) (layer "B.Cu") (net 55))
 (segment (start 190.759 45.212) (end 176.134 45.212) (width 2) (layer "B.Cu") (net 56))
 (segment (start 143.256 126.852) (end 143.256 115.824) (width 1) (layer "B.Cu") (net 27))
 (segment (start 140.716 113.284) (end 143.256 115.824) (width 1) (layer "B.Cu") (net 27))
 (segment (start 131.064 113.284) (end 140.716 113.284) (width 1) (layer "B.Cu") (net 27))
 (segment (start 137.414 130.81) (end 142.748 130.81) (width 1) (layer "B.Cu") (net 39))
 (segment (start 144.526 129.032) (end 144.526 126.852) (width 1) (layer "B.Cu") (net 39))
 (segment (start 142.748 130.81) (end 144.526 129.032) (width 1) (layer "B.Cu") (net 39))
 (segment (start 214.63 124.206) (end 214.63 74.168) (width 1) (layer "B.Cu") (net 41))
 (segment (start 213.36 125.476) (end 214.63 124.206) (width 1) (layer "B.Cu") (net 41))
 (segment (start 198.12 128.778) (end 203.962 128.778) (width 1) (layer "B.Cu") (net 41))
 (segment (start 214.63 74.168) (end 202.946 62.484) (width 1) (layer "B.Cu") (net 41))
 (segment (start 203.962 128.778) (end 207.264 125.476) (width 1) (layer "B.Cu") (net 41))
 (segment (start 207.264 125.476) (end 211.399 125.476) (width 1) (layer "B.Cu") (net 41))
 (segment (start 211.399 125.476) (end 213.36 125.476) (width 1) (layer "B.Cu") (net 41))
 (segment (start 131.064 108.204) (end 142.24 108.204) (width 1) (layer "B.Cu") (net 29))
 (segment (start 151.384 117.348) (end 151.384 121.666) (width 1) (layer "B.Cu") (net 29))
 (segment (start 151.384 121.666) (end 151.384 126.238) (width 1) (layer "B.Cu") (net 29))
 (segment (start 142.24 108.204) (end 151.384 117.348) (width 1) (layer "B.Cu") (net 29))
 (segment (start 174.264 121.666) (end 174.508 121.91) (width 1) (layer "B.Cu") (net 46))
 (segment (start 161.544 121.666) (end 174.264 121.666) (width 1) (layer "B.Cu") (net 46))
 (segment (start 194.828 121.91) (end 198.12 118.618) (width 1) (layer "B.Cu") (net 49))
 (segment (start 182.128 121.91) (end 194.828 121.91) (width 1) (layer "B.Cu") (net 49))
 (segment (start 208.788 45.183) (end 193.328 45.183) (width 2) (layer "B.Cu") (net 43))
 (segment (start 193.328 45.183) (end 193.299 45.212) (width 2) (layer "B.Cu") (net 43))
 (segment (start 98.22 116.156) (end 90.424 116.156) (width 1) (layer "B.Cu") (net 11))
 (segment (start 108.204 110.744) (end 103.632 110.744) (width 1) (layer "B.Cu") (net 11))
 (segment (start 103.632 110.744) (end 98.22 116.156) (width 1) (layer "B.Cu") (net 11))
 (segment (start 100.584 103.886) (end 100.506 103.964) (width 1) (layer "B.Cu") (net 10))
 (segment (start 100.506 103.964) (end 90.678 103.964) (width 1) (layer "B.Cu") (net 10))
 (segment (start 108.204 108.204) (end 104.902 108.204) (width 1) (layer "B.Cu") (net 10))
 (segment (start 104.902 108.204) (end 100.584 103.886) (width 1) (layer "B.Cu") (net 10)))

